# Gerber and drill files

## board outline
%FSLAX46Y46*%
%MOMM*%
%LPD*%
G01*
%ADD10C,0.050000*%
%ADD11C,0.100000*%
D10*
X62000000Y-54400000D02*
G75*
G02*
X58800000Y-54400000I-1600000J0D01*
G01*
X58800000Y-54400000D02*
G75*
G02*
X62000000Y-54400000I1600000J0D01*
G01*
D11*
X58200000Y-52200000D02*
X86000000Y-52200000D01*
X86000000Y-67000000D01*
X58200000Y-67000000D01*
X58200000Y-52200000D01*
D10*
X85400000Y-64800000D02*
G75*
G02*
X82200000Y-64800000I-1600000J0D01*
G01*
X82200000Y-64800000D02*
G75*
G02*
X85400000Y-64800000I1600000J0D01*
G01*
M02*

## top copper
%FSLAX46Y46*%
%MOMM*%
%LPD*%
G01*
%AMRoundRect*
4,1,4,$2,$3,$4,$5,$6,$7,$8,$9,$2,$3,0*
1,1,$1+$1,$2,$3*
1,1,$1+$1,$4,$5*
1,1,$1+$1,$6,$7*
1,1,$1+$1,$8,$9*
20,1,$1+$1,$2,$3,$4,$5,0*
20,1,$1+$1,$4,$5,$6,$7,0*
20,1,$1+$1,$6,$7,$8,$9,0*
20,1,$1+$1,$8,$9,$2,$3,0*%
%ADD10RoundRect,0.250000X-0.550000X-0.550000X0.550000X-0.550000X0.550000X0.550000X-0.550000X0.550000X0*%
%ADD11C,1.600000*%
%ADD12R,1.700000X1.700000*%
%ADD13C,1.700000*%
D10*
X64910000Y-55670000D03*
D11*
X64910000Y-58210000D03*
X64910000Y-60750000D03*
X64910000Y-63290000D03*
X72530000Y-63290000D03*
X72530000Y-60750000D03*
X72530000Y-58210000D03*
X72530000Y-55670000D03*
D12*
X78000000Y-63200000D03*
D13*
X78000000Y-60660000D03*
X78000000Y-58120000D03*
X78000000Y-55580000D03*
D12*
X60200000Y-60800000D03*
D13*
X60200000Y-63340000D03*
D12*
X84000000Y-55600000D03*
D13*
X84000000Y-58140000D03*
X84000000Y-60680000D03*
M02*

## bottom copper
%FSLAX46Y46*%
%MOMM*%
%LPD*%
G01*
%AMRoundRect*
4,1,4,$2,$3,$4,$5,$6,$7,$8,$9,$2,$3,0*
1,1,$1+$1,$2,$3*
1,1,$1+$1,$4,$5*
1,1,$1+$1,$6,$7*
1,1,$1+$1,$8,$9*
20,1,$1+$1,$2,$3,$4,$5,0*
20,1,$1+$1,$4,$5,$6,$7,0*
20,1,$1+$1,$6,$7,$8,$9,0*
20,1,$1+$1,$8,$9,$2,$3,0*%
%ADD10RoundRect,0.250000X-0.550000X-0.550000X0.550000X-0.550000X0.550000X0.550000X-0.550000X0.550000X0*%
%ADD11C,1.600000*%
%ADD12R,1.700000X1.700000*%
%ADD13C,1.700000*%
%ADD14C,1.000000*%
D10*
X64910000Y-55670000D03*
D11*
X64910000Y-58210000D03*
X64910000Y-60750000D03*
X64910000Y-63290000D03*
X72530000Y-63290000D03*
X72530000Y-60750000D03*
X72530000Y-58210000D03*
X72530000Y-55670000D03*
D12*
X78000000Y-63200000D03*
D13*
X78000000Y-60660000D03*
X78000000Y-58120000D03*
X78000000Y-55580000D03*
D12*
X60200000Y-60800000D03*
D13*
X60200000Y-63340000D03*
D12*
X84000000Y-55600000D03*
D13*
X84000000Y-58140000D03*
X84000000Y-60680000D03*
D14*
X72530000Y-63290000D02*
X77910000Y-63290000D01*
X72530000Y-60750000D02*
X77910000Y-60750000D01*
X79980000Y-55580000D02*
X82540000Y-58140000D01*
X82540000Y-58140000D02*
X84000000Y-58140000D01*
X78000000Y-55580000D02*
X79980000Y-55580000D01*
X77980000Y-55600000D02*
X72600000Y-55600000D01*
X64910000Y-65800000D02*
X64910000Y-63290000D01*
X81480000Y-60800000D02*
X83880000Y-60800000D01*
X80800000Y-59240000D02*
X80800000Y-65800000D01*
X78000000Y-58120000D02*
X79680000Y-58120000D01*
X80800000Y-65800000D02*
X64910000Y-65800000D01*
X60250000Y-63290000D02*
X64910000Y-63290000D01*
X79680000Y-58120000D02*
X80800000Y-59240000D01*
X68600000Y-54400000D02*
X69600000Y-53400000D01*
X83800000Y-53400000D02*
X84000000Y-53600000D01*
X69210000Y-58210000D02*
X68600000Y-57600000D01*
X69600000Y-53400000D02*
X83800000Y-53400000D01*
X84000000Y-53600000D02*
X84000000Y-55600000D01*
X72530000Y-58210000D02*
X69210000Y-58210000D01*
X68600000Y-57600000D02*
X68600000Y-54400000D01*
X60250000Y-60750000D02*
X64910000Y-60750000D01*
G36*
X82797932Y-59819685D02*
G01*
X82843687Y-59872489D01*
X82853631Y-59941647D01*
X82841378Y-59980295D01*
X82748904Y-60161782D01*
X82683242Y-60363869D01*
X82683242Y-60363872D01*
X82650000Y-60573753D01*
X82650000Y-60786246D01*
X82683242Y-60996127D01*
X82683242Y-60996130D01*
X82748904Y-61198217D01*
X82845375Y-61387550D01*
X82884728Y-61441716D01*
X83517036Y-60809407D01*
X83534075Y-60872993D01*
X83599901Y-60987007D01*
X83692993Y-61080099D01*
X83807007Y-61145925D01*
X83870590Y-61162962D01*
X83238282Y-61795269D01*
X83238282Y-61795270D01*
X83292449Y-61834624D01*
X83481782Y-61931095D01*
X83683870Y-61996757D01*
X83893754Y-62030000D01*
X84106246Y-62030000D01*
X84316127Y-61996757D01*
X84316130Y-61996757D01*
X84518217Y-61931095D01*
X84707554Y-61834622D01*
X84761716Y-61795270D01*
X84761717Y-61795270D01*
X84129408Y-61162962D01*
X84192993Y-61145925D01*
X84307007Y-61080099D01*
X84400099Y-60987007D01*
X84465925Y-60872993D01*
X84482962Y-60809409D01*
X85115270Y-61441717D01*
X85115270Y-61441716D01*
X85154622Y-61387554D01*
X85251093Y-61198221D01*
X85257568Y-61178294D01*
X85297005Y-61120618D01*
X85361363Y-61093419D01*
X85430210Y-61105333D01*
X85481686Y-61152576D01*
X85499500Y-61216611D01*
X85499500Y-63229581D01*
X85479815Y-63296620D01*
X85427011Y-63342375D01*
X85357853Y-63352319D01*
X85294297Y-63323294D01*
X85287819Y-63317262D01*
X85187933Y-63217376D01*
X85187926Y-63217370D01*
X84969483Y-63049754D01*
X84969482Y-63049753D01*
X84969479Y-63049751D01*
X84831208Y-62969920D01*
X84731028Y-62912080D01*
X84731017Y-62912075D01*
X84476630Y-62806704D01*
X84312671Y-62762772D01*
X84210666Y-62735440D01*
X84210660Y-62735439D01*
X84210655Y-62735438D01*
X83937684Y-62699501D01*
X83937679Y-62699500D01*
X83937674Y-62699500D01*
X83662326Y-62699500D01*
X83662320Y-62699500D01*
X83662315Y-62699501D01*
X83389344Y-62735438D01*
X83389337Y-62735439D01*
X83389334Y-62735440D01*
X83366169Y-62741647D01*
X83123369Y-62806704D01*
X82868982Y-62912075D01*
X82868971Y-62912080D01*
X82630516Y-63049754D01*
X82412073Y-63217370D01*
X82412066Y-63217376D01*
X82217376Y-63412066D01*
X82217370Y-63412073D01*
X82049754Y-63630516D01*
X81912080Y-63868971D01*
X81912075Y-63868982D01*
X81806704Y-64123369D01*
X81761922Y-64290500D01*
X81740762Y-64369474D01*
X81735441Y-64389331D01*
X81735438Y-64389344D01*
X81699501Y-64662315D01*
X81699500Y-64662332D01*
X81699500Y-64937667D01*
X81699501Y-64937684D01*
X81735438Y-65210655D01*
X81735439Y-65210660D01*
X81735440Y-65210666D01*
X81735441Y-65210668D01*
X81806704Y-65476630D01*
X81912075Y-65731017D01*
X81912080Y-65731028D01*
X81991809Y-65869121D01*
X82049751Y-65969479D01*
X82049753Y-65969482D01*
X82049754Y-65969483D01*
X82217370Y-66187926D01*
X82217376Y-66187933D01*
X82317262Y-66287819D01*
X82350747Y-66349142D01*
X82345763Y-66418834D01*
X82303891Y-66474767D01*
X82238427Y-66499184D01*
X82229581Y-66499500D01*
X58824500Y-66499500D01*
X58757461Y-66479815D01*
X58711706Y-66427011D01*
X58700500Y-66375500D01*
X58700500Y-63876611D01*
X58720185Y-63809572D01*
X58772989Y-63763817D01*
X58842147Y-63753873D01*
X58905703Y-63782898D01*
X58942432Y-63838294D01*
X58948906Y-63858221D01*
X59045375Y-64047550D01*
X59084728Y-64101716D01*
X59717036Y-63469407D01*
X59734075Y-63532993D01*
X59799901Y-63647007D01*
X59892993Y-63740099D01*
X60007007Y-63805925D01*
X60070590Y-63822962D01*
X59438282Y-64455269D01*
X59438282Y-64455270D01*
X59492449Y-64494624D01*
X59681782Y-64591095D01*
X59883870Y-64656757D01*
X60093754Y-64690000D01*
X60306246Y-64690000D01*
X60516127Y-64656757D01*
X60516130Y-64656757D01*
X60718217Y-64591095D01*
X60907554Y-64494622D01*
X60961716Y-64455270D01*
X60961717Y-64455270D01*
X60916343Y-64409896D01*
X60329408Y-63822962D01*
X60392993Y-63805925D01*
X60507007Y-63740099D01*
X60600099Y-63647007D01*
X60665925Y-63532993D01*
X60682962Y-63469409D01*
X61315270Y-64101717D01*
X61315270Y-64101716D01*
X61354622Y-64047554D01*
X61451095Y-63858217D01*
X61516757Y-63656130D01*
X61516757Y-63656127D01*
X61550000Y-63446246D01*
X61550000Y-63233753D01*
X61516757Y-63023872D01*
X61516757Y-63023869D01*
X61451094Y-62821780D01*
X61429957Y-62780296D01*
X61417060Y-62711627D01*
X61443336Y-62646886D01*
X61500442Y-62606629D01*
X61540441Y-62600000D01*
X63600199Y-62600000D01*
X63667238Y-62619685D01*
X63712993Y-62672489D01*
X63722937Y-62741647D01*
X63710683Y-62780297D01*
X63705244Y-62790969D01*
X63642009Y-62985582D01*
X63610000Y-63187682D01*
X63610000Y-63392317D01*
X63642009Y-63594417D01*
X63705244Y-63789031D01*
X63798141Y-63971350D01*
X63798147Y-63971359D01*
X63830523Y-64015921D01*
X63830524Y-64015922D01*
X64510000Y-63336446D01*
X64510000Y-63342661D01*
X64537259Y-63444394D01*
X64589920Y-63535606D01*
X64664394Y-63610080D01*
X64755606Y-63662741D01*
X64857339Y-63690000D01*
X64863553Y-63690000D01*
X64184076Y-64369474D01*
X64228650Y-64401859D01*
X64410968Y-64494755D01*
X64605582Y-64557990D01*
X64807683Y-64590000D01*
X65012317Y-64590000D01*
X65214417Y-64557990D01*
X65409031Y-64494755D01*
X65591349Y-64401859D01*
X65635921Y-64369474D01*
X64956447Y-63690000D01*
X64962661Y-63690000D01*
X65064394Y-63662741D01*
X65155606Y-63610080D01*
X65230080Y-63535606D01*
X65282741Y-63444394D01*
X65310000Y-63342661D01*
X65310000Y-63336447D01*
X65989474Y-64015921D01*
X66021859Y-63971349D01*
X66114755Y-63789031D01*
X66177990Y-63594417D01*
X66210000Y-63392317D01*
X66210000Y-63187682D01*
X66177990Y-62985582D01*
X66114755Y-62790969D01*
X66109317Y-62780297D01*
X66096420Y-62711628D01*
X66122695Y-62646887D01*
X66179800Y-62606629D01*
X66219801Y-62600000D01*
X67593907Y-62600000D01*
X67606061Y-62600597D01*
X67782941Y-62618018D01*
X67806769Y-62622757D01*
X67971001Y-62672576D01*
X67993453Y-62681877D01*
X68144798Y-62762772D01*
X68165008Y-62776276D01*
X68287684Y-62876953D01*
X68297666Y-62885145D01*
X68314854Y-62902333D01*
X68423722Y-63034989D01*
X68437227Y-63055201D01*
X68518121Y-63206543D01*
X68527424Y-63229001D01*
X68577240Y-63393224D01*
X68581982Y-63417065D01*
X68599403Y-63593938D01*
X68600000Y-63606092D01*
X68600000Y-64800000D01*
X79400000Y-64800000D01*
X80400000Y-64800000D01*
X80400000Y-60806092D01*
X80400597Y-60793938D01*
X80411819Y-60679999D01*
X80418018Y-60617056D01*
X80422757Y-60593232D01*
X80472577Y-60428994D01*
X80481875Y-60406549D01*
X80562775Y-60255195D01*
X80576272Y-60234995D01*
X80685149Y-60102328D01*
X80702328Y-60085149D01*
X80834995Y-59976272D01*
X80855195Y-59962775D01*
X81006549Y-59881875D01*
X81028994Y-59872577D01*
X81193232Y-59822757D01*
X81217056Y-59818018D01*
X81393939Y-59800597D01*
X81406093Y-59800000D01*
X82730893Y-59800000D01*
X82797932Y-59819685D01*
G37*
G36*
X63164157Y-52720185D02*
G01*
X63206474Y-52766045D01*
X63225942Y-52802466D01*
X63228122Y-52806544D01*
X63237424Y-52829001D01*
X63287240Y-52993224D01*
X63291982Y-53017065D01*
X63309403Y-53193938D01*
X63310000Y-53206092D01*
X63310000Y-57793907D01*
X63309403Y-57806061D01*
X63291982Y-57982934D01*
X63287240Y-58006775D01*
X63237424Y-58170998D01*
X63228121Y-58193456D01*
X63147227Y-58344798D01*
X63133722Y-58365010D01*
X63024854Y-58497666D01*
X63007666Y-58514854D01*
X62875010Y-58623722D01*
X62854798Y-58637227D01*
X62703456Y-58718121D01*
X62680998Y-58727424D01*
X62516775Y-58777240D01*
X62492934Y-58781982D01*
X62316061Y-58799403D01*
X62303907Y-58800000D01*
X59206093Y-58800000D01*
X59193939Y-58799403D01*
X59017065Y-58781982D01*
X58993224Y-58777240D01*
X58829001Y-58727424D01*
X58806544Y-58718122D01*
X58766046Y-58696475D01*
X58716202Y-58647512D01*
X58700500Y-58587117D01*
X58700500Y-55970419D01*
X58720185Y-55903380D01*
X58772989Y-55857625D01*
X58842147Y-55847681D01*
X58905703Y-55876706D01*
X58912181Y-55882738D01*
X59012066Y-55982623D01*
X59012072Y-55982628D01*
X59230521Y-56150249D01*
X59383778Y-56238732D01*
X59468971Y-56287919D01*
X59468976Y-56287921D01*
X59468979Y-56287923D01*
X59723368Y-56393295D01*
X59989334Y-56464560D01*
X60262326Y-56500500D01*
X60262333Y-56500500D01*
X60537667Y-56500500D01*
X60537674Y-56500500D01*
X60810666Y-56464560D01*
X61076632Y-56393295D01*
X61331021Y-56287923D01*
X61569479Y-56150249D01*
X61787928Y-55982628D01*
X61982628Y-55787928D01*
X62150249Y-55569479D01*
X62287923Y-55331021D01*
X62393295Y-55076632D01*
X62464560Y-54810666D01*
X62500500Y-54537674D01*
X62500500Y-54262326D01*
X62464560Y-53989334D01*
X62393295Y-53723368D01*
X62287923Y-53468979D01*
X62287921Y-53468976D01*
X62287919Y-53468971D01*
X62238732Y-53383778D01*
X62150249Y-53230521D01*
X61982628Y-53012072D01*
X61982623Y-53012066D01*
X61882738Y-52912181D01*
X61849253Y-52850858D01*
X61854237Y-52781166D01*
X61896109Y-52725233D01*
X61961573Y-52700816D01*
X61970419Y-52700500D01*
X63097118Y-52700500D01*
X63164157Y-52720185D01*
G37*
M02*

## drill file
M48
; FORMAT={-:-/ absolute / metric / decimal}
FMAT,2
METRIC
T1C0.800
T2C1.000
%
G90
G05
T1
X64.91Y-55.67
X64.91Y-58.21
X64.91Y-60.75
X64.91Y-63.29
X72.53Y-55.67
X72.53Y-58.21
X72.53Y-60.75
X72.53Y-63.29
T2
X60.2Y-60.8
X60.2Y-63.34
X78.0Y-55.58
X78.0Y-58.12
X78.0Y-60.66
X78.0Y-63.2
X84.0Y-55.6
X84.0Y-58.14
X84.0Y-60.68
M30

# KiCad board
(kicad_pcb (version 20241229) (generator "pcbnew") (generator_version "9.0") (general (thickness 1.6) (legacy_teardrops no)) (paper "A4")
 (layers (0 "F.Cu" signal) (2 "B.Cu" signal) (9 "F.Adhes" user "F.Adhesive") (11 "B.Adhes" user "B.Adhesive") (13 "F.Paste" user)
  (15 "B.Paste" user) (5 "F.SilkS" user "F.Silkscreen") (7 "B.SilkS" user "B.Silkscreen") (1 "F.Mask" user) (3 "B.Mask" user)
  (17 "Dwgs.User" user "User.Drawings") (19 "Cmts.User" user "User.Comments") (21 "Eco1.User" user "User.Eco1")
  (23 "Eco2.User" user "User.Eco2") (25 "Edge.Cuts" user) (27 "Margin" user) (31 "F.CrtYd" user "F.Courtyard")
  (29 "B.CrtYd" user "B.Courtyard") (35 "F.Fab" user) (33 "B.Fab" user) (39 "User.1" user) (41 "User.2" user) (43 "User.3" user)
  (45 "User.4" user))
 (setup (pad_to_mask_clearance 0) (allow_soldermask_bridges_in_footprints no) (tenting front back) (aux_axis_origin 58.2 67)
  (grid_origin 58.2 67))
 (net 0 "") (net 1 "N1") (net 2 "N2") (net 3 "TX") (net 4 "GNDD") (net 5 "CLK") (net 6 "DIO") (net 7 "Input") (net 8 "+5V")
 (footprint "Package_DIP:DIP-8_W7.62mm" (layer "F.Cu") (at 64.91 55.67)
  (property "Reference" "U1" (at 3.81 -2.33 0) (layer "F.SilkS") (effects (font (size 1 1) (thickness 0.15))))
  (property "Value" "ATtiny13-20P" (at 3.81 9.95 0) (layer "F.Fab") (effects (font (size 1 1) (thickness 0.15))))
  (pad "1" thru_hole roundrect (at 0 0) (size 1.6 1.6) (drill 0.8) (layers "*.Cu" "*.Mask") (remove_unused_layers no)
   (roundrect_rratio 0.15625) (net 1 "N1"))
  (pad "2" thru_hole circle (at 0 2.54) (size 1.6 1.6) (drill 0.8) (layers "*.Cu" "*.Mask") (remove_unused_layers no) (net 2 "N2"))
  (pad "3" thru_hole circle (at 0 5.08) (size 1.6 1.6) (drill 0.8) (layers "*.Cu" "*.Mask") (remove_unused_layers no) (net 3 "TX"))
  (pad "4" thru_hole circle (at 0 7.62) (size 1.6 1.6) (drill 0.8) (layers "*.Cu" "*.Mask") (remove_unused_layers no) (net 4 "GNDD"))
  (pad "5" thru_hole circle (at 7.62 7.62) (size 1.6 1.6) (drill 0.8) (layers "*.Cu" "*.Mask") (remove_unused_layers no) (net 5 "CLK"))
  (pad "6" thru_hole circle (at 7.62 5.08) (size 1.6 1.6) (drill 0.8) (layers "*.Cu" "*.Mask") (remove_unused_layers no) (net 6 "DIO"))
  (pad "7" thru_hole circle (at 7.62 2.54) (size 1.6 1.6) (drill 0.8) (layers "*.Cu" "*.Mask") (remove_unused_layers no) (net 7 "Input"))
  (pad "8" thru_hole circle (at 7.62 0) (size 1.6 1.6) (drill 0.8) (layers "*.Cu" "*.Mask") (remove_unused_layers no) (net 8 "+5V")))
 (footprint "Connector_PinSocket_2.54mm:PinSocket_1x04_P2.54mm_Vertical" (layer "F.Cu") (at 78 63.2 180)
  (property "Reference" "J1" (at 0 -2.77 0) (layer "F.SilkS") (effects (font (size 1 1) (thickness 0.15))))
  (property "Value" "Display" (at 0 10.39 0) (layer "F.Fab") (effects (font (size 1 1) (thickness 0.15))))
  (pad "1" thru_hole rect (at 0 0 180) (size 1.7 1.7) (drill 1) (layers "*.Cu" "*.Mask") (remove_unused_layers no) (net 5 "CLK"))
  (pad "2" thru_hole circle (at 0 2.54 180) (size 1.7 1.7) (drill 1) (layers "*.Cu" "*.Mask") (remove_unused_layers no) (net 6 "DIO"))
  (pad "3" thru_hole circle (at 0 5.08 180) (size 1.7 1.7) (drill 1) (layers "*.Cu" "*.Mask") (remove_unused_layers no) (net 4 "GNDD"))
  (pad "4" thru_hole circle (at 0 7.62 180) (size 1.7 1.7) (drill 1) (layers "*.Cu" "*.Mask") (remove_unused_layers no) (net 8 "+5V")))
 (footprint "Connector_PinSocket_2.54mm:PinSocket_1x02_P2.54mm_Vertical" (layer "F.Cu") (at 60.2 60.8)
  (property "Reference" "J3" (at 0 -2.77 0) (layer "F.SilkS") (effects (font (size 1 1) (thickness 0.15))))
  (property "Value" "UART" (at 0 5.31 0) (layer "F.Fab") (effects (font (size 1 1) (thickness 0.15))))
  (pad "1" thru_hole rect (at 0 0) (size 1.7 1.7) (drill 1) (layers "*.Cu" "*.Mask") (remove_unused_layers no) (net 3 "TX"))
  (pad "2" thru_hole circle (at 0 2.54) (size 1.7 1.7) (drill 1) (layers "*.Cu" "*.Mask") (remove_unused_layers no) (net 4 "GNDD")))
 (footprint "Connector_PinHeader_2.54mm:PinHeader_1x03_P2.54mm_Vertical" (layer "F.Cu") (at 84 55.6)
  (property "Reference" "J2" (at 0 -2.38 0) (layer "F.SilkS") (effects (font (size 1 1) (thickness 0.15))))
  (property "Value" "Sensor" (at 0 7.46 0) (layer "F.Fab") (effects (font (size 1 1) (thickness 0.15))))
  (pad "1" thru_hole rect (at 0 0) (size 1.7 1.7) (drill 1) (layers "*.Cu" "*.Mask") (remove_unused_layers no) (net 7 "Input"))
  (pad "2" thru_hole circle (at 0 2.54) (size 1.7 1.7) (drill 1) (layers "*.Cu" "*.Mask") (remove_unused_layers no) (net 8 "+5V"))
  (pad "3" thru_hole circle (at 0 5.08) (size 1.7 1.7) (drill 1) (layers "*.Cu" "*.Mask") (remove_unused_layers no) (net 4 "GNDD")))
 (gr_circle (center 60.4 54.4) (end 62 54.4) (stroke (width 0.05) (type solid)) (fill no) (layer "Edge.Cuts"))
 (gr_rect (start 58.2 52.2) (end 86 67) (stroke (width 0.1) (type solid)) (fill no) (layer "Edge.Cuts"))
 (gr_circle (center 83.8 64.8) (end 85.4 64.8) (stroke (width 0.05) (type solid)) (fill no) (layer "Edge.Cuts"))
 (segment (start 72.53 63.29) (end 77.91 63.29) (width 1) (layer "B.Cu") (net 5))
 (segment (start 72.53 60.75) (end 77.91 60.75) (width 1) (layer "B.Cu") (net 6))
 (segment (start 79.98 55.58) (end 82.54 58.14) (width 1) (layer "B.Cu") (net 8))
 (segment (start 82.54 58.14) (end 84 58.14) (width 1) (layer "B.Cu") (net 8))
 (segment (start 78 55.58) (end 79.98 55.58) (width 1) (layer "B.Cu") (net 8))
 (segment (start 77.98 55.6) (end 72.6 55.6) (width 1) (layer "B.Cu") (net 8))
 (segment (start 64.91 65.8) (end 64.91 63.29) (width 1) (layer "B.Cu") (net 4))
 (segment (start 81.48 60.8) (end 83.88 60.8) (width 1) (layer "B.Cu") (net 4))
 (segment (start 80.8 59.24) (end 80.8 65.8) (width 1) (layer "B.Cu") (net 4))
 (segment (start 78 58.12) (end 79.68 58.12) (width 1) (layer "B.Cu") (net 4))
 (segment (start 80.8 65.8) (end 64.91 65.8) (width 1) (layer "B.Cu") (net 4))
 (segment (start 60.25 63.29) (end 64.91 63.29) (width 1) (layer "B.Cu") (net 4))
 (segment (start 79.68 58.12) (end 80.8 59.24) (width 1) (layer "B.Cu") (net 4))
 (segment (start 68.6 54.4) (end 69.6 53.4) (width 1) (layer "B.Cu") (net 7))
 (segment (start 83.8 53.4) (end 84 53.6) (width 1) (layer "B.Cu") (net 7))
 (segment (start 69.21 58.21) (end 68.6 57.6) (width 1) (layer "B.Cu") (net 7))
 (segment (start 69.6 53.4) (end 83.8 53.4) (width 1) (layer "B.Cu") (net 7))
 (segment (start 84 53.6) (end 84 55.6) (width 1) (layer "B.Cu") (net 7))
 (segment (start 72.53 58.21) (end 69.21 58.21) (width 1) (layer "B.Cu") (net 7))
 (segment (start 68.6 57.6) (end 68.6 54.4) (width 1) (layer "B.Cu") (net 7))
 (segment (start 60.25 60.75) (end 64.91 60.75) (width 1) (layer "B.Cu") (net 3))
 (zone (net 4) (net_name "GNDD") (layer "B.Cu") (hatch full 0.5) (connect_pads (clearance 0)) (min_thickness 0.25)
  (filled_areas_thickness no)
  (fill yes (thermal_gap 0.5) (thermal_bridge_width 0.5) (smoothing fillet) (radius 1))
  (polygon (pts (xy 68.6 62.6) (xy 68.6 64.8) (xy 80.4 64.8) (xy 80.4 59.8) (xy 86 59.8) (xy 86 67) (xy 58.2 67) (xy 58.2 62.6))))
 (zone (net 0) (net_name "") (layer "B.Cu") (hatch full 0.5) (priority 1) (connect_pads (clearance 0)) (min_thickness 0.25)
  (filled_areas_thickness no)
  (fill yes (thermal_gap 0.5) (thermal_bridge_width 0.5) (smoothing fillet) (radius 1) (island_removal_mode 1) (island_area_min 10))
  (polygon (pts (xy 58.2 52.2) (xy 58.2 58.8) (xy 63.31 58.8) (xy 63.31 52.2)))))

